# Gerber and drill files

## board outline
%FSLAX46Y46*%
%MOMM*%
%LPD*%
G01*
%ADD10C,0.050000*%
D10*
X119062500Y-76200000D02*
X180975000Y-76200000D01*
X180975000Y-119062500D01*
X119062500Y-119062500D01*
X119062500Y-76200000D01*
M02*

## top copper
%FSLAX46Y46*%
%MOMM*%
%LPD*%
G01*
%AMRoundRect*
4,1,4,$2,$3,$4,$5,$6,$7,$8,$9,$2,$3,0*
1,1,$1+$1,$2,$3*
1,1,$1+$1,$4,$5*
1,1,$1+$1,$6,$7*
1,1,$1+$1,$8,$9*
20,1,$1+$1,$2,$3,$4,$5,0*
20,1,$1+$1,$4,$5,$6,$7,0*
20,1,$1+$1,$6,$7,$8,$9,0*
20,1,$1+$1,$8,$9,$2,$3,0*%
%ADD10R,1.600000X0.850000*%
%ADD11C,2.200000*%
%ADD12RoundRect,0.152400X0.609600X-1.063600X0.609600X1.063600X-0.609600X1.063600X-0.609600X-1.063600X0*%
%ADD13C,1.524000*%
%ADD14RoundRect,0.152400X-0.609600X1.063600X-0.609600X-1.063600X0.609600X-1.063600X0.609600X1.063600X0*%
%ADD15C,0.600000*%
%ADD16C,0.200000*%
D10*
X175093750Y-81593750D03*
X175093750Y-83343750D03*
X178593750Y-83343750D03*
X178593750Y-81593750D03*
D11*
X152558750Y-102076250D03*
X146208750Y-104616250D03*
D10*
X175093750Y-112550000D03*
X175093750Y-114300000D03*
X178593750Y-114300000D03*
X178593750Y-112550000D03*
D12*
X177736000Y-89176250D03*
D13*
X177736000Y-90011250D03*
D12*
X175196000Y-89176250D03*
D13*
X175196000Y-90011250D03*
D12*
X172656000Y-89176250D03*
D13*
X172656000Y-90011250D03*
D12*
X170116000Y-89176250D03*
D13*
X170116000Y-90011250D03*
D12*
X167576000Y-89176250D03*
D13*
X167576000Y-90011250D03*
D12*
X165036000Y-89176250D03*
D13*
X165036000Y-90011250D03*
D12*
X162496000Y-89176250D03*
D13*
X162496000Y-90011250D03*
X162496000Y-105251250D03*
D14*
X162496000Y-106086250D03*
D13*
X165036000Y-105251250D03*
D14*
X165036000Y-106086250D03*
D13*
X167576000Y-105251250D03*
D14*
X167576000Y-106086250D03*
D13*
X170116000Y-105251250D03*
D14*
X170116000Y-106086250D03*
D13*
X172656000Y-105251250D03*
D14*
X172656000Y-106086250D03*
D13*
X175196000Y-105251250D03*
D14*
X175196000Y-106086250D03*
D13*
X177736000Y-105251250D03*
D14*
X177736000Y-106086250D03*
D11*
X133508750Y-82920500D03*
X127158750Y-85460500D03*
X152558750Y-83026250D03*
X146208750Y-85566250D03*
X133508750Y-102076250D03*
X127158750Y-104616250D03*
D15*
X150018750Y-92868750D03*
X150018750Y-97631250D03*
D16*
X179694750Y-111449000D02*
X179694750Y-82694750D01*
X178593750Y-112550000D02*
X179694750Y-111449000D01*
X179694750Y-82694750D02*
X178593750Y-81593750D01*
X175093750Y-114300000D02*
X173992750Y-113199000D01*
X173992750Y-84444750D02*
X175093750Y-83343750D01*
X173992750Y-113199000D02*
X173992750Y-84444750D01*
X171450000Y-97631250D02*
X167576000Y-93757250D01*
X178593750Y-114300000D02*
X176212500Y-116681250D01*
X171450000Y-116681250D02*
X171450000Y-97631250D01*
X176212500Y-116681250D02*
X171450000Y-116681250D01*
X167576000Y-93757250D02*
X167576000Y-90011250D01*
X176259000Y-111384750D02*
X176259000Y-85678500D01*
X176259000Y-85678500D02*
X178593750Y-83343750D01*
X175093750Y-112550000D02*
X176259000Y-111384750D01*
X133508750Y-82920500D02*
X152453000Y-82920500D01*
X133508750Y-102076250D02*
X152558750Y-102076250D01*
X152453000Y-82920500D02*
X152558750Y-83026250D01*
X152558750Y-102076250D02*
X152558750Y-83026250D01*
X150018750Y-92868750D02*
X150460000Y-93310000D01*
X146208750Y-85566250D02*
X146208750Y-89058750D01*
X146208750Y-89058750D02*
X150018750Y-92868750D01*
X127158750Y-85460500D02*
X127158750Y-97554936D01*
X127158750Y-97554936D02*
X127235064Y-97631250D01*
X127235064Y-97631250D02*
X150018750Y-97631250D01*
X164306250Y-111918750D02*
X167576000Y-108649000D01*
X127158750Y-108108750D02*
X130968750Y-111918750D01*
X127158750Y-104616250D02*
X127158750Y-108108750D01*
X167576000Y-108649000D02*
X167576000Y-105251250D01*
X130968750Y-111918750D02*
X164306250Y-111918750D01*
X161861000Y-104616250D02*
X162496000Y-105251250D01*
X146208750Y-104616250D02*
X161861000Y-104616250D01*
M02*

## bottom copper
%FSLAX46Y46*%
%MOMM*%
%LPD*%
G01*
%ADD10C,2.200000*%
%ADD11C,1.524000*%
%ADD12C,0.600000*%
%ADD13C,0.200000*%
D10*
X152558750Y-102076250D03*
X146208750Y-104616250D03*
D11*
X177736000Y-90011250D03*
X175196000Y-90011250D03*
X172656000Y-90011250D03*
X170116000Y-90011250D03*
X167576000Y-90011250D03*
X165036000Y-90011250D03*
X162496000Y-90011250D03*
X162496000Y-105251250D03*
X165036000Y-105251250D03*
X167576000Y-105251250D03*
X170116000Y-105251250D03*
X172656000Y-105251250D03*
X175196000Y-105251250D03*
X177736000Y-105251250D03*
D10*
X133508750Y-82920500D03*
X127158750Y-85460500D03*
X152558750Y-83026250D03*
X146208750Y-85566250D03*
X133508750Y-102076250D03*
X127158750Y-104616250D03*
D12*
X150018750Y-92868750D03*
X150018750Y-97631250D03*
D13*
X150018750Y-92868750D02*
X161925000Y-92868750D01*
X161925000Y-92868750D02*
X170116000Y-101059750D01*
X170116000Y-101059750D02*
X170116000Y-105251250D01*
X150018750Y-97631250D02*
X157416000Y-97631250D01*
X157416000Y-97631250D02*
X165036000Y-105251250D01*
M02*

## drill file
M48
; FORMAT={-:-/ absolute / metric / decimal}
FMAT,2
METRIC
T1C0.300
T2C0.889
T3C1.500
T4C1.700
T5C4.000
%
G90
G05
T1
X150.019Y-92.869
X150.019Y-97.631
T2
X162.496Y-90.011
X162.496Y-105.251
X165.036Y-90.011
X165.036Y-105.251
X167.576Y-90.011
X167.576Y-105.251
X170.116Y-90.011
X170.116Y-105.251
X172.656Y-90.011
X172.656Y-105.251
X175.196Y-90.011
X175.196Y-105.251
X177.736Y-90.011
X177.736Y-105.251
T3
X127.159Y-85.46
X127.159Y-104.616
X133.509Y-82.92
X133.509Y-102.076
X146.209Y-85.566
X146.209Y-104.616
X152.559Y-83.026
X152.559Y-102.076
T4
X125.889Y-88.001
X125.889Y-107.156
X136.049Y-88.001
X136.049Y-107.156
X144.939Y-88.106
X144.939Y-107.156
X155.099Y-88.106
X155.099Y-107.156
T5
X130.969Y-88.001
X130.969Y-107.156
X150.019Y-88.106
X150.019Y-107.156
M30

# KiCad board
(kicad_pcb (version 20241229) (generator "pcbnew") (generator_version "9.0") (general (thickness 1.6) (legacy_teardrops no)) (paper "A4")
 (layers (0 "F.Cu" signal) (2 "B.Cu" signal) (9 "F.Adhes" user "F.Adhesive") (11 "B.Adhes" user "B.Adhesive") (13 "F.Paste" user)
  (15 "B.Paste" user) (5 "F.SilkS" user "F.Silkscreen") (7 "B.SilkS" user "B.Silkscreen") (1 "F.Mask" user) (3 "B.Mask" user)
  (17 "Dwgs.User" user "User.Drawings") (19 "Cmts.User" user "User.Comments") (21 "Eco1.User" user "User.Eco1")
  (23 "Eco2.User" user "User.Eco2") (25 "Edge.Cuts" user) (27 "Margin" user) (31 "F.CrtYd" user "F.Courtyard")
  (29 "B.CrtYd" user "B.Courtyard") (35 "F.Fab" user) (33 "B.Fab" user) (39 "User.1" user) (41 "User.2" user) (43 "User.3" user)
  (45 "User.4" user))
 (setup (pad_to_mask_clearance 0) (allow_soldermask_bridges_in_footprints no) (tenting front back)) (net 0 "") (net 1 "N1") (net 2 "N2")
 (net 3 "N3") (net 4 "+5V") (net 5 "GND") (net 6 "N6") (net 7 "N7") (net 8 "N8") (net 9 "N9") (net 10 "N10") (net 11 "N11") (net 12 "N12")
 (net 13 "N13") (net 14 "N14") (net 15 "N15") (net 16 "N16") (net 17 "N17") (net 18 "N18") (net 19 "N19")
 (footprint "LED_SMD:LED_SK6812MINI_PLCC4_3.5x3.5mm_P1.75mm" (layer "F.Cu") (at 176.84375 82.46875)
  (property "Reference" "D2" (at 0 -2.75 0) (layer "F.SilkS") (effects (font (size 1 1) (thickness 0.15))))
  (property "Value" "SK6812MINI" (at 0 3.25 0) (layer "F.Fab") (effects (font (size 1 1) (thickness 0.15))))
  (pad "1" smd rect (at -1.75 -0.875) (size 1.6 0.85) (layers "F.Cu" "F.Mask" "F.Paste") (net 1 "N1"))
  (pad "2" smd rect (at -1.75 0.875) (size 1.6 0.85) (layers "F.Cu" "F.Mask" "F.Paste") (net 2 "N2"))
  (pad "3" smd rect (at 1.75 0.875) (size 1.6 0.85) (layers "F.Cu" "F.Mask" "F.Paste") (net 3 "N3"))
  (pad "4" smd rect (at 1.75 -0.875) (size 1.6 0.85) (layers "F.Cu" "F.Mask" "F.Paste") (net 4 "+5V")))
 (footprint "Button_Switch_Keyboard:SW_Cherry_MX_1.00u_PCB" (layer "F.Cu") (at 152.55875 102.07625)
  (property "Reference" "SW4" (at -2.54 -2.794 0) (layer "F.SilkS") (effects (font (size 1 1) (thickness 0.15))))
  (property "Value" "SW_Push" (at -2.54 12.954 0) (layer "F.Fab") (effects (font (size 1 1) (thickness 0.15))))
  (pad "" np_thru_hole circle (at -7.62 5.08) (size 1.7 1.7) (drill 1.7) (layers "*.Cu" "*.Mask"))
  (pad "" np_thru_hole circle (at -2.54 5.08) (size 4 4) (drill 4) (layers "*.Cu" "*.Mask"))
  (pad "" np_thru_hole circle (at 2.54 5.08) (size 1.7 1.7) (drill 1.7) (layers "*.Cu" "*.Mask"))
  (pad "1" thru_hole circle (at 0 0) (size 2.2 2.2) (drill 1.5) (layers "*.Cu" "*.Mask") (remove_unused_layers no) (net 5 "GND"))
  (pad "2" thru_hole circle (at -6.35 2.54) (size 2.2 2.2) (drill 1.5) (layers "*.Cu" "*.Mask") (remove_unused_layers no) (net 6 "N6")))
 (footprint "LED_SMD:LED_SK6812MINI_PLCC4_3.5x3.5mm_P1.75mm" (layer "F.Cu") (at 176.84375 113.425)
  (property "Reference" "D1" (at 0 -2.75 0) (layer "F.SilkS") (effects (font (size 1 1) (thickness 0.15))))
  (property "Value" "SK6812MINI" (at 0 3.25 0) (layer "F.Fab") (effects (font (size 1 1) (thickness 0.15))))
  (pad "1" smd rect (at -1.75 -0.875) (size 1.6 0.85) (layers "F.Cu" "F.Mask" "F.Paste") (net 3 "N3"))
  (pad "2" smd rect (at -1.75 0.875) (size 1.6 0.85) (layers "F.Cu" "F.Mask" "F.Paste") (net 2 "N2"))
  (pad "3" smd rect (at 1.75 0.875) (size 1.6 0.85) (layers "F.Cu" "F.Mask" "F.Paste") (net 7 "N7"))
  (pad "4" smd rect (at 1.75 -0.875) (size 1.6 0.85) (layers "F.Cu" "F.Mask" "F.Paste") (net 4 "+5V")))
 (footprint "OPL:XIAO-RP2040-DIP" (layer "F.Cu") (at 170.116 97.63125 -90)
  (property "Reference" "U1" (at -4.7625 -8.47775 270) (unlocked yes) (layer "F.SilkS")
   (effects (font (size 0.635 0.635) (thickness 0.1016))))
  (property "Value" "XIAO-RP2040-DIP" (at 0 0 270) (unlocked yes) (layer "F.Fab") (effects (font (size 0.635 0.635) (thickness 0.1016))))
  (pad "1" smd roundrect (at -8.455 -7.62 90) (size 2.432 1.524) (layers "F.Cu" "F.Mask") (roundrect_rratio 0.1) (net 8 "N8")
   (thermal_bridge_angle 45))
  (pad "1" thru_hole circle (at -7.62 -7.62 90) (size 1.524 1.524) (drill 0.889) (layers "*.Cu" "*.Mask") (remove_unused_layers no)
   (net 8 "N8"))
  (pad "2" smd roundrect (at -8.455 -5.08 90) (size 2.432 1.524) (layers "F.Cu" "F.Mask") (roundrect_rratio 0.1) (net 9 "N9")
   (thermal_bridge_angle 45))
  (pad "2" thru_hole circle (at -7.62 -5.08 90) (size 1.524 1.524) (drill 0.889) (layers "*.Cu" "*.Mask") (remove_unused_layers no)
   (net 9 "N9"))
  (pad "3" smd roundrect (at -8.455 -2.54 90) (size 2.432 1.524) (layers "F.Cu" "F.Mask") (roundrect_rratio 0.1) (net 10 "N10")
   (thermal_bridge_angle 45))
  (pad "3" thru_hole circle (at -7.62 -2.54 90) (size 1.524 1.524) (drill 0.889) (layers "*.Cu" "*.Mask") (remove_unused_layers no)
   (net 10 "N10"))
  (pad "4" smd roundrect (at -8.455 0 90) (size 2.432 1.524) (layers "F.Cu" "F.Mask") (roundrect_rratio 0.1) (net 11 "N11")
   (thermal_bridge_angle 45))
  (pad "4" thru_hole circle (at -7.62 0 90) (size 1.524 1.524) (drill 0.889) (layers "*.Cu" "*.Mask") (remove_unused_layers no)
   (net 11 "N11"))
  (pad "5" smd roundrect (at -8.455 2.54 90) (size 2.432 1.524) (layers "F.Cu" "F.Mask") (roundrect_rratio 0.1) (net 7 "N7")
   (thermal_bridge_angle 45))
  (pad "5" thru_hole circle (at -7.62 2.54 90) (size 1.524 1.524) (drill 0.889) (layers "*.Cu" "*.Mask") (remove_unused_layers no)
   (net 7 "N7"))
  (pad "6" smd roundrect (at -8.455 5.08 90) (size 2.432 1.524) (layers "F.Cu" "F.Mask") (roundrect_rratio 0.1) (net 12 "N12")
   (thermal_bridge_angle 45))
  (pad "6" thru_hole circle (at -7.62 5.08 90) (size 1.524 1.524) (drill 0.889) (layers "*.Cu" "*.Mask") (remove_unused_layers no)
   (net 12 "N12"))
  (pad "7" smd roundrect (at -8.455 7.62 90) (size 2.432 1.524) (layers "F.Cu" "F.Mask") (roundrect_rratio 0.1) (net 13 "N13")
   (thermal_bridge_angle 45))
  (pad "7" thru_hole circle (at -7.62 7.62 90) (size 1.524 1.524) (drill 0.889) (layers "*.Cu" "*.Mask") (remove_unused_layers no)
   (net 13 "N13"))
  (pad "8" thru_hole circle (at 7.62 7.62 270) (size 1.524 1.524) (drill 0.889) (layers "*.Cu" "*.Mask") (remove_unused_layers no)
   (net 6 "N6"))
  (pad "8" smd roundrect (at 8.455 7.62 270) (size 2.432 1.524) (layers "F.Cu" "F.Mask") (roundrect_rratio 0.1) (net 6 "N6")
   (thermal_bridge_angle 45))
  (pad "9" thru_hole circle (at 7.62 5.08 270) (size 1.524 1.524) (drill 0.889) (layers "*.Cu" "*.Mask") (remove_unused_layers no)
   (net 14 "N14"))
  (pad "9" smd roundrect (at 8.455 5.08 270) (size 2.432 1.524) (layers "F.Cu" "F.Mask") (roundrect_rratio 0.1) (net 14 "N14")
   (thermal_bridge_angle 45))
  (pad "10" thru_hole circle (at 7.62 2.54 270) (size 1.524 1.524) (drill 0.889) (layers "*.Cu" "*.Mask") (remove_unused_layers no)
   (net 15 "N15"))
  (pad "10" smd roundrect (at 8.455 2.54 270) (size 2.432 1.524) (layers "F.Cu" "F.Mask") (roundrect_rratio 0.1) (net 15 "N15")
   (thermal_bridge_angle 45))
  (pad "11" thru_hole circle (at 7.62 0 270) (size 1.524 1.524) (drill 0.889) (layers "*.Cu" "*.Mask") (remove_unused_layers no)
   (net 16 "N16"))
  (pad "11" smd roundrect (at 8.455 0 270) (size 2.432 1.524) (layers "F.Cu" "F.Mask") (roundrect_rratio 0.1) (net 16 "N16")
   (thermal_bridge_angle 45))
  (pad "12" thru_hole circle (at 7.62 -2.54 270) (size 1.524 1.524) (drill 0.889) (layers "*.Cu" "*.Mask") (remove_unused_layers no)
   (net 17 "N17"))
  (pad "12" smd roundrect (at 8.455 -2.54 270) (size 2.432 1.524) (layers "F.Cu" "F.Mask") (roundrect_rratio 0.1) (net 17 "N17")
   (thermal_bridge_angle 45))
  (pad "13" thru_hole circle (at 7.62 -5.08 270) (size 1.524 1.524) (drill 0.889) (layers "*.Cu" "*.Mask") (remove_unused_layers no)
   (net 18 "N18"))
  (pad "13" smd roundrect (at 8.455 -5.08 270) (size 2.432 1.524) (layers "F.Cu" "F.Mask") (roundrect_rratio 0.1) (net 18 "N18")
   (thermal_bridge_angle 45))
  (pad "14" thru_hole circle (at 7.62 -7.62 270) (size 1.524 1.524) (drill 0.889) (layers "*.Cu" "*.Mask") (remove_unused_layers no)
   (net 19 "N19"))
  (pad "14" smd roundrect (at 8.455 -7.62 270) (size 2.432 1.524) (layers "F.Cu" "F.Mask") (roundrect_rratio 0.1) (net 19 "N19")
   (thermal_bridge_angle 45)))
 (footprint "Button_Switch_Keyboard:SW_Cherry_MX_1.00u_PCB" (layer "F.Cu") (at 133.50875 82.9205)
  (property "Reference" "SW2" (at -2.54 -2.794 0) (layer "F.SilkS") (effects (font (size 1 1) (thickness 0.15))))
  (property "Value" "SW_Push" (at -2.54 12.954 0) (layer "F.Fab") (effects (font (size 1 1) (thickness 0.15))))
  (pad "" np_thru_hole circle (at -7.62 5.08) (size 1.7 1.7) (drill 1.7) (layers "*.Cu" "*.Mask"))
  (pad "" np_thru_hole circle (at -2.54 5.08) (size 4 4) (drill 4) (layers "*.Cu" "*.Mask"))
  (pad "" np_thru_hole circle (at 2.54 5.08) (size 1.7 1.7) (drill 1.7) (layers "*.Cu" "*.Mask"))
  (pad "1" thru_hole circle (at 0 0) (size 2.2 2.2) (drill 1.5) (layers "*.Cu" "*.Mask") (remove_unused_layers no) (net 5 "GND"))
  (pad "2" thru_hole circle (at -6.35 2.54) (size 2.2 2.2) (drill 1.5) (layers "*.Cu" "*.Mask") (remove_unused_layers no) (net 14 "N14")))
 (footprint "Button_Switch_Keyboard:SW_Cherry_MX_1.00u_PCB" (layer "F.Cu") (at 152.55875 83.02625)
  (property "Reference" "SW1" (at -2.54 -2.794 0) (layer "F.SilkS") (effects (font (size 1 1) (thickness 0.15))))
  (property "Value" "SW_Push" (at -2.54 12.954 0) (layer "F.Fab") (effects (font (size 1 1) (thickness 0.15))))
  (pad "" np_thru_hole circle (at -7.62 5.08) (size 1.7 1.7) (drill 1.7) (layers "*.Cu" "*.Mask"))
  (pad "" np_thru_hole circle (at -2.54 5.08) (size 4 4) (drill 4) (layers "*.Cu" "*.Mask"))
  (pad "" np_thru_hole circle (at 2.54 5.08) (size 1.7 1.7) (drill 1.7) (layers "*.Cu" "*.Mask"))
  (pad "1" thru_hole circle (at 0 0) (size 2.2 2.2) (drill 1.5) (layers "*.Cu" "*.Mask") (remove_unused_layers no) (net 5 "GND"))
  (pad "2" thru_hole circle (at -6.35 2.54) (size 2.2 2.2) (drill 1.5) (layers "*.Cu" "*.Mask") (remove_unused_layers no) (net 16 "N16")))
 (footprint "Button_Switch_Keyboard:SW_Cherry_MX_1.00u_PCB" (layer "F.Cu") (at 133.50875 102.07625)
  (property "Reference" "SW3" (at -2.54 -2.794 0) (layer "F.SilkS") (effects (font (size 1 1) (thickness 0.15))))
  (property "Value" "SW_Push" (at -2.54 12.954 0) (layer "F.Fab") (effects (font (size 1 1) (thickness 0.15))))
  (pad "" np_thru_hole circle (at -7.62 5.08) (size 1.7 1.7) (drill 1.7) (layers "*.Cu" "*.Mask"))
  (pad "" np_thru_hole circle (at -2.54 5.08) (size 4 4) (drill 4) (layers "*.Cu" "*.Mask"))
  (pad "" np_thru_hole circle (at 2.54 5.08) (size 1.7 1.7) (drill 1.7) (layers "*.Cu" "*.Mask"))
  (pad "1" thru_hole circle (at 0 0) (size 2.2 2.2) (drill 1.5) (layers "*.Cu" "*.Mask") (remove_unused_layers no) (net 5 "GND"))
  (pad "2" thru_hole circle (at -6.35 2.54) (size 2.2 2.2) (drill 1.5) (layers "*.Cu" "*.Mask") (remove_unused_layers no) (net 15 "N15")))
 (gr_rect (start 119.0625 76.2) (end 180.975 119.0625) (stroke (width 0.05) (type default)) (fill no) (layer "Edge.Cuts"))
 (segment (start 179.69475 111.449) (end 179.69475 82.69475) (width 0.2) (layer "F.Cu") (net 4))
 (segment (start 178.59375 112.55) (end 179.69475 111.449) (width 0.2) (layer "F.Cu") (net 4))
 (segment (start 179.69475 82.69475) (end 178.59375 81.59375) (width 0.2) (layer "F.Cu") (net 4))
 (segment (start 175.09375 114.3) (end 173.99275 113.199) (width 0.2) (layer "F.Cu") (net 2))
 (segment (start 173.99275 84.44475) (end 175.09375 83.34375) (width 0.2) (layer "F.Cu") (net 2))
 (segment (start 173.99275 113.199) (end 173.99275 84.44475) (width 0.2) (layer "F.Cu") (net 2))
 (segment (start 171.45 97.63125) (end 167.576 93.75725) (width 0.2) (layer "F.Cu") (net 7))
 (segment (start 178.59375 114.3) (end 176.2125 116.68125) (width 0.2) (layer "F.Cu") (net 7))
 (segment (start 171.45 116.68125) (end 171.45 97.63125) (width 0.2) (layer "F.Cu") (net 7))
 (segment (start 176.2125 116.68125) (end 171.45 116.68125) (width 0.2) (layer "F.Cu") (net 7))
 (segment (start 167.576 93.75725) (end 167.576 90.01125) (width 0.2) (layer "F.Cu") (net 7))
 (segment (start 176.259 111.38475) (end 176.259 85.6785) (width 0.2) (layer "F.Cu") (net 3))
 (segment (start 176.259 85.6785) (end 178.59375 83.34375) (width 0.2) (layer "F.Cu") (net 3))
 (segment (start 175.09375 112.55) (end 176.259 111.38475) (width 0.2) (layer "F.Cu") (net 3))
 (segment (start 133.50875 82.9205) (end 152.453 82.9205) (width 0.2) (layer "F.Cu") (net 5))
 (segment (start 133.50875 102.07625) (end 152.55875 102.07625) (width 0.2) (layer "F.Cu") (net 5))
 (segment (start 152.453 82.9205) (end 152.55875 83.02625) (width 0.2) (layer "F.Cu") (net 5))
 (segment (start 152.55875 102.07625) (end 152.55875 83.02625) (width 0.2) (layer "F.Cu") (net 5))
 (segment (start 150.01875 92.86875) (end 150.46 93.31) (width 0.2) (layer "F.Cu") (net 16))
 (segment (start 146.20875 85.56625) (end 146.20875 89.05875) (width 0.2) (layer "F.Cu") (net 16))
 (segment (start 146.20875 89.05875) (end 150.01875 92.86875) (width 0.2) (layer "F.Cu") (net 16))
 (via (at 150.01875 92.86875) (size 0.6) (drill 0.3) (layers "F.Cu" "B.Cu") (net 16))
 (segment (start 150.01875 92.86875) (end 161.925 92.86875) (width 0.2) (layer "B.Cu") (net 16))
 (segment (start 161.925 92.86875) (end 170.116 101.05975) (width 0.2) (layer "B.Cu") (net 16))
 (segment (start 170.116 101.05975) (end 170.116 105.25125) (width 0.2) (layer "B.Cu") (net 16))
 (segment (start 127.15875 85.4605) (end 127.15875 97.554936) (width 0.2) (layer "F.Cu") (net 14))
 (segment (start 127.15875 97.554936) (end 127.235064 97.63125) (width 0.2) (layer "F.Cu") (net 14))
 (segment (start 127.235064 97.63125) (end 150.01875 97.63125) (width 0.2) (layer "F.Cu") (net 14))
 (via (at 150.01875 97.63125) (size 0.6) (drill 0.3) (layers "F.Cu" "B.Cu") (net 14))
 (segment (start 150.01875 97.63125) (end 157.416 97.63125) (width 0.2) (layer "B.Cu") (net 14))
 (segment (start 157.416 97.63125) (end 165.036 105.25125) (width 0.2) (layer "B.Cu") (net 14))
 (segment (start 164.30625 111.91875) (end 167.576 108.649) (width 0.2) (layer "F.Cu") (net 15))
 (segment (start 127.15875 108.10875) (end 130.96875 111.91875) (width 0.2) (layer "F.Cu") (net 15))
 (segment (start 127.15875 104.61625) (end 127.15875 108.10875) (width 0.2) (layer "F.Cu") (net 15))
 (segment (start 167.576 108.649) (end 167.576 105.25125) (width 0.2) (layer "F.Cu") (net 15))
 (segment (start 130.96875 111.91875) (end 164.30625 111.91875) (width 0.2) (layer "F.Cu") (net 15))
 (segment (start 161.861 104.61625) (end 162.496 105.25125) (width 0.2) (layer "F.Cu") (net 6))
 (segment (start 146.20875 104.61625) (end 161.861 104.61625) (width 0.2) (layer "F.Cu") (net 6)))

